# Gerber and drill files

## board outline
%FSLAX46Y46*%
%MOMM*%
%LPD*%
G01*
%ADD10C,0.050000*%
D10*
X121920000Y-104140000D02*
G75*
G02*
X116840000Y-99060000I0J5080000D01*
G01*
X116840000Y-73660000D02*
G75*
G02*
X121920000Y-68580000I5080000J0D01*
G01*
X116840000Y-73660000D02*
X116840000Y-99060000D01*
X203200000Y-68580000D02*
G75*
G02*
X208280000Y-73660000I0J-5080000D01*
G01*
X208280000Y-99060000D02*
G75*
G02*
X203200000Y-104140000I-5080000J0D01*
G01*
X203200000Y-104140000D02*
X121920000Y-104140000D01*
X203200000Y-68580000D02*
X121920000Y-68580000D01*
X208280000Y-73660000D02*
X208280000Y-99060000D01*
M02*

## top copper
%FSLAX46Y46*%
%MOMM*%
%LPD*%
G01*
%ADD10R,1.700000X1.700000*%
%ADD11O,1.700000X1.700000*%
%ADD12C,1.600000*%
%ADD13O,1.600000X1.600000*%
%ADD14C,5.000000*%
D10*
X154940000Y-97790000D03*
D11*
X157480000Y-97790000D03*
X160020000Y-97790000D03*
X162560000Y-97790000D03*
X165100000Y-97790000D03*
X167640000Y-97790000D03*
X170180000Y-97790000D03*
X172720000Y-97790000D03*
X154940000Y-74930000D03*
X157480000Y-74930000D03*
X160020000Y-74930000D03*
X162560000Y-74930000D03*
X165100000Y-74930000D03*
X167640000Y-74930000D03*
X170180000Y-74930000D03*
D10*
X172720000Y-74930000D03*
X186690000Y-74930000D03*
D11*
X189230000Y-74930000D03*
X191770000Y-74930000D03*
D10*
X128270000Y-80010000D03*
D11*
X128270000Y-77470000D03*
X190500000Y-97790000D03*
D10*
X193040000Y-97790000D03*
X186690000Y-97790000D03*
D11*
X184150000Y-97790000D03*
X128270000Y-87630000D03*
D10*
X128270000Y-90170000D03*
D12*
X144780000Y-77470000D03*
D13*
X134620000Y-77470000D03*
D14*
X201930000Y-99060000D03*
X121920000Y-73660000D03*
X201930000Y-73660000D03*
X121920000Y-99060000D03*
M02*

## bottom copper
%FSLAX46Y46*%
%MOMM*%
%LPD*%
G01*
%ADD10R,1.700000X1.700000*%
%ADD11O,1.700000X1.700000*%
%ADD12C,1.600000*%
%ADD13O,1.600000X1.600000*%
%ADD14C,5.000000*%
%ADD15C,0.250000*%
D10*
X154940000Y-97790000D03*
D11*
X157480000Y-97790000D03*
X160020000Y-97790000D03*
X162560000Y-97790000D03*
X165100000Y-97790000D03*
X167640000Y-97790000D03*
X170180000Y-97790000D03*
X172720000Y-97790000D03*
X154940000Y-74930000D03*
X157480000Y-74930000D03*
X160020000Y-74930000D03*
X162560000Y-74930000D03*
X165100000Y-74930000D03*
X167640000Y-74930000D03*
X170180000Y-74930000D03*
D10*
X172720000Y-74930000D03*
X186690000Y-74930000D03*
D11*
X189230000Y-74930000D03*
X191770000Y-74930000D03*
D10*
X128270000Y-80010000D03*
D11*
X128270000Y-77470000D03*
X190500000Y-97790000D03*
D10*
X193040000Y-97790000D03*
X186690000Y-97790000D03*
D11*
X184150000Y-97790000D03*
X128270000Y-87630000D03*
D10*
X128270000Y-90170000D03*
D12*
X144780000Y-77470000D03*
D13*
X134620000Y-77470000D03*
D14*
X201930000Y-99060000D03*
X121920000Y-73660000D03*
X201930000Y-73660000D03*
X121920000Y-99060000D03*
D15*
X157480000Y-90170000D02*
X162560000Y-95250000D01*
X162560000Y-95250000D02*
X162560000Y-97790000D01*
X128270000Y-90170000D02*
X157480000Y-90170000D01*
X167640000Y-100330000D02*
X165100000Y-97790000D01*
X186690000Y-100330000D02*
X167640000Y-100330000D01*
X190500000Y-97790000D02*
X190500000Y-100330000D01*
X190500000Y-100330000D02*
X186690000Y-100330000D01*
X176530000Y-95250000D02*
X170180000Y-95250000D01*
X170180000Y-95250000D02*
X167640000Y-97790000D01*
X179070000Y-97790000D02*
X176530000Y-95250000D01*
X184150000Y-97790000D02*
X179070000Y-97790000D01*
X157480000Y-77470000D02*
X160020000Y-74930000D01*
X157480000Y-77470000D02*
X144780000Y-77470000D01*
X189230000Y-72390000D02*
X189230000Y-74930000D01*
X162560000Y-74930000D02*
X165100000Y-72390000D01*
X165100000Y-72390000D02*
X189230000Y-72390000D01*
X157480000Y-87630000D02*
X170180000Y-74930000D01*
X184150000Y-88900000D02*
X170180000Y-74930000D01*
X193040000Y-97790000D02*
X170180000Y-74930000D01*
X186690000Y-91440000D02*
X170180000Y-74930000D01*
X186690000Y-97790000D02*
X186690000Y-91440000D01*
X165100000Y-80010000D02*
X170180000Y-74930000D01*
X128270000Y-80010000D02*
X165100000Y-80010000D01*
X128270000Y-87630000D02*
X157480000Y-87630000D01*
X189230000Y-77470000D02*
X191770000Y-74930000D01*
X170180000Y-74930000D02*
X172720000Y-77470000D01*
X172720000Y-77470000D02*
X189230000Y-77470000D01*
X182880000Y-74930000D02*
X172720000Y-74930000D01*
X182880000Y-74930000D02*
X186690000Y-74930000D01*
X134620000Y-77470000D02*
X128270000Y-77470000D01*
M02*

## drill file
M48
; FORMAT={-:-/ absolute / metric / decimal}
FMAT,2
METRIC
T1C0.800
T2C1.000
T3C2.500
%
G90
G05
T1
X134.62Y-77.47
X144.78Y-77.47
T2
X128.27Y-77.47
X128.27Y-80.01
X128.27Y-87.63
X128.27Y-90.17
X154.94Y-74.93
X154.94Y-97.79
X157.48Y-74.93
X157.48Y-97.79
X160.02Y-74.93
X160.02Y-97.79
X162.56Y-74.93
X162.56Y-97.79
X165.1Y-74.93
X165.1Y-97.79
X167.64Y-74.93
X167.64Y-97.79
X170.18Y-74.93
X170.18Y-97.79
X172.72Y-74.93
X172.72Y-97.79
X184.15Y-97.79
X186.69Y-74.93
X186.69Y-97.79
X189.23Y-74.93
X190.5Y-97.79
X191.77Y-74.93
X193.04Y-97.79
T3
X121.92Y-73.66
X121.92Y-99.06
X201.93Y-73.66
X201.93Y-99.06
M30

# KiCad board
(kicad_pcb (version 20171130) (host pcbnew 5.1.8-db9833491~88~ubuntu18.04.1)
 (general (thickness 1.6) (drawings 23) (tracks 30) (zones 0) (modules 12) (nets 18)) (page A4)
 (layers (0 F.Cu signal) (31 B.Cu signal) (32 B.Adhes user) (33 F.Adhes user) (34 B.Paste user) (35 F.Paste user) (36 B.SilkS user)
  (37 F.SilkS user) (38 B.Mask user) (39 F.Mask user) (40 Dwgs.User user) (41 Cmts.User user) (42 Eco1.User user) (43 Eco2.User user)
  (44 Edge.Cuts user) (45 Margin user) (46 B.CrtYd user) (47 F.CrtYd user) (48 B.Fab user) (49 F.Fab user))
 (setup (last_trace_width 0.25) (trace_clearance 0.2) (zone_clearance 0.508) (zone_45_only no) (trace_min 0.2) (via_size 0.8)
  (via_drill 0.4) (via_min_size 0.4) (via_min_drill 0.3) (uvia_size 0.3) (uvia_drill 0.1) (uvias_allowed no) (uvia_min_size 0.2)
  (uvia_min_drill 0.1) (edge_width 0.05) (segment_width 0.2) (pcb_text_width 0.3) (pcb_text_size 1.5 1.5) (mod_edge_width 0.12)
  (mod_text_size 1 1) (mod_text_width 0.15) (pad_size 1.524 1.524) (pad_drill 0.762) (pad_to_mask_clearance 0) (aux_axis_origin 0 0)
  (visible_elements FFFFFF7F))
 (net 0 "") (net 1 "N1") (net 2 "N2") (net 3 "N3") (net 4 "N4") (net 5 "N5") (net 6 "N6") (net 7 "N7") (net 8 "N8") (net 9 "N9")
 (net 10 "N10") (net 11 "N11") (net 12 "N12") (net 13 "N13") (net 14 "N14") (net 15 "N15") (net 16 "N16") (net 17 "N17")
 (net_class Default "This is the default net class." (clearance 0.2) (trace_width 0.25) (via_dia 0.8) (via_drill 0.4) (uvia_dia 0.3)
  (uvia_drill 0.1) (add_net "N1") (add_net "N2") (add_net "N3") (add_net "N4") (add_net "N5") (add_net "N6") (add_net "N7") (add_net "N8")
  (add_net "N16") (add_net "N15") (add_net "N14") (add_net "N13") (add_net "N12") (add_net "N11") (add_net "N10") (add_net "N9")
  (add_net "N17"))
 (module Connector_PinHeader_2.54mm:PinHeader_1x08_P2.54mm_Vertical (layer F.Cu) (at 154.94 97.79 90)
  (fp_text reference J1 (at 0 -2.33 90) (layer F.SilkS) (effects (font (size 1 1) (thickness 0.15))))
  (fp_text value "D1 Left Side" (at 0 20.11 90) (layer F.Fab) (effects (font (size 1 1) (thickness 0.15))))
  (pad 1 thru_hole rect (at 0 0 90) (size 1.7 1.7) (drill 1) (layers *.Cu *.Mask) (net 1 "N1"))
  (pad 2 thru_hole oval (at 0 2.54 90) (size 1.7 1.7) (drill 1) (layers *.Cu *.Mask) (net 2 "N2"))
  (pad 3 thru_hole oval (at 0 5.08 90) (size 1.7 1.7) (drill 1) (layers *.Cu *.Mask) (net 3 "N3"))
  (pad 4 thru_hole oval (at 0 7.62 90) (size 1.7 1.7) (drill 1) (layers *.Cu *.Mask) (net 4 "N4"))
  (pad 5 thru_hole oval (at 0 10.16 90) (size 1.7 1.7) (drill 1) (layers *.Cu *.Mask) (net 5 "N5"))
  (pad 6 thru_hole oval (at 0 12.7 90) (size 1.7 1.7) (drill 1) (layers *.Cu *.Mask) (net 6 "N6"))
  (pad 7 thru_hole oval (at 0 15.24 90) (size 1.7 1.7) (drill 1) (layers *.Cu *.Mask) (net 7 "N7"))
  (pad 8 thru_hole oval (at 0 17.78 90) (size 1.7 1.7) (drill 1) (layers *.Cu *.Mask) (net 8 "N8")))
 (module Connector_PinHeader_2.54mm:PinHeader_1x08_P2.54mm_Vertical (layer F.Cu) (at 172.72 74.93 270)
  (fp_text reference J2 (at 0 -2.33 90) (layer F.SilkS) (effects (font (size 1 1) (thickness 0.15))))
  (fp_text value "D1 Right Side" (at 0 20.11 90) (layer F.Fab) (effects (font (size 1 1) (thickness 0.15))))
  (pad 8 thru_hole oval (at 0 17.78 270) (size 1.7 1.7) (drill 1) (layers *.Cu *.Mask) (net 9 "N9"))
  (pad 7 thru_hole oval (at 0 15.24 270) (size 1.7 1.7) (drill 1) (layers *.Cu *.Mask) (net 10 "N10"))
  (pad 6 thru_hole oval (at 0 12.7 270) (size 1.7 1.7) (drill 1) (layers *.Cu *.Mask) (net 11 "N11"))
  (pad 5 thru_hole oval (at 0 10.16 270) (size 1.7 1.7) (drill 1) (layers *.Cu *.Mask) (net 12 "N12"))
  (pad 4 thru_hole oval (at 0 7.62 270) (size 1.7 1.7) (drill 1) (layers *.Cu *.Mask) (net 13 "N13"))
  (pad 3 thru_hole oval (at 0 5.08 270) (size 1.7 1.7) (drill 1) (layers *.Cu *.Mask) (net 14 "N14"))
  (pad 2 thru_hole oval (at 0 2.54 270) (size 1.7 1.7) (drill 1) (layers *.Cu *.Mask) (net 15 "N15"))
  (pad 1 thru_hole rect (at 0 0 270) (size 1.7 1.7) (drill 1) (layers *.Cu *.Mask) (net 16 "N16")))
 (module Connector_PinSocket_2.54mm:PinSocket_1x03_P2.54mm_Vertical (layer F.Cu) (at 186.69 74.93 90)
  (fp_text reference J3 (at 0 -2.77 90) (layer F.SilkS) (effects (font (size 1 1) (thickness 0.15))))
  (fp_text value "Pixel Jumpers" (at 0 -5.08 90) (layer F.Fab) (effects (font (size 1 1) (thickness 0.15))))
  (pad 1 thru_hole rect (at 0 0 90) (size 1.7 1.7) (drill 1) (layers *.Cu *.Mask) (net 16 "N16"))
  (pad 2 thru_hole oval (at 0 2.54 90) (size 1.7 1.7) (drill 1) (layers *.Cu *.Mask) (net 12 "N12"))
  (pad 3 thru_hole oval (at 0 5.08 90) (size 1.7 1.7) (drill 1) (layers *.Cu *.Mask) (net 15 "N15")))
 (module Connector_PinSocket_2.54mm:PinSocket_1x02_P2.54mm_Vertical (layer F.Cu) (at 128.27 80.01 180)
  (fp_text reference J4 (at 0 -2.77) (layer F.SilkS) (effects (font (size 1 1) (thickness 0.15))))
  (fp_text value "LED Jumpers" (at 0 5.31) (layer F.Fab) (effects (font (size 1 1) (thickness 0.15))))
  (pad 1 thru_hole rect (at 0 0 180) (size 1.7 1.7) (drill 1) (layers *.Cu *.Mask) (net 15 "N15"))
  (pad 2 thru_hole oval (at 0 2.54 180) (size 1.7 1.7) (drill 1) (layers *.Cu *.Mask) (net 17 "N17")))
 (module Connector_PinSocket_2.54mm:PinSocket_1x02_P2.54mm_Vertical (layer F.Cu) (at 193.04 97.79 270)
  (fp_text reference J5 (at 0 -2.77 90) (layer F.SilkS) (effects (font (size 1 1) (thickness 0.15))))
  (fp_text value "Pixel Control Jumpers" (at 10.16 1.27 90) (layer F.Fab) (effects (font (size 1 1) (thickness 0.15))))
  (pad 2 thru_hole oval (at 0 2.54 270) (size 1.7 1.7) (drill 1) (layers *.Cu *.Mask) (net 5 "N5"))
  (pad 1 thru_hole rect (at 0 0 270) (size 1.7 1.7) (drill 1) (layers *.Cu *.Mask) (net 15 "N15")))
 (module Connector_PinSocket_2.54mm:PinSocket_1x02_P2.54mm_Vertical (layer F.Cu) (at 186.69 97.79 270)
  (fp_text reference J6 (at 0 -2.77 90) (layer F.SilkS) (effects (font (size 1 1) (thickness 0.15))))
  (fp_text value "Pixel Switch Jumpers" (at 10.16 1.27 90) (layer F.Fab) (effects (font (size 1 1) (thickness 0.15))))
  (pad 1 thru_hole rect (at 0 0 270) (size 1.7 1.7) (drill 1) (layers *.Cu *.Mask) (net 15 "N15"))
  (pad 2 thru_hole oval (at 0 2.54 270) (size 1.7 1.7) (drill 1) (layers *.Cu *.Mask) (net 6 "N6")))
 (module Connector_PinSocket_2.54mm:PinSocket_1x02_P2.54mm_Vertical (layer F.Cu) (at 128.27 90.17 180)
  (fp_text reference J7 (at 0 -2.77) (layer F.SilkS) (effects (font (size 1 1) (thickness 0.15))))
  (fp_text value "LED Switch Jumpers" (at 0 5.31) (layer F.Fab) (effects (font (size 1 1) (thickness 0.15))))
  (pad 2 thru_hole oval (at 0 2.54 180) (size 1.7 1.7) (drill 1) (layers *.Cu *.Mask) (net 15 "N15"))
  (pad 1 thru_hole rect (at 0 0 180) (size 1.7 1.7) (drill 1) (layers *.Cu *.Mask) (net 4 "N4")))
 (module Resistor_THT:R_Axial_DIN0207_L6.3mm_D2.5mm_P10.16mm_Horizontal (layer F.Cu) (at 144.78 77.47 180)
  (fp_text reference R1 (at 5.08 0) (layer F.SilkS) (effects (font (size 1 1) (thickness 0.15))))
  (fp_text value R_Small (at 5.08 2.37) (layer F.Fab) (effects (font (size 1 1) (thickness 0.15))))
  (pad 1 thru_hole circle (at 0 0 180) (size 1.6 1.6) (drill 0.8) (layers *.Cu *.Mask) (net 11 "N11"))
  (pad 2 thru_hole oval (at 10.16 0 180) (size 1.6 1.6) (drill 0.8) (layers *.Cu *.Mask) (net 17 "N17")))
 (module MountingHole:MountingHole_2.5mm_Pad (layer F.Cu) (at 201.93 99.06)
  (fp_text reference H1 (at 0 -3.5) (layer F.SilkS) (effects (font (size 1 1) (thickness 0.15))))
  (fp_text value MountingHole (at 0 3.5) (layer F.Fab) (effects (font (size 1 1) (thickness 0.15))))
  (pad 1 thru_hole circle (at 0 0) (size 5 5) (drill 2.5) (layers *.Cu *.Mask)))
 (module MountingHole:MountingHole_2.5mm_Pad (layer F.Cu) (at 121.92 73.66)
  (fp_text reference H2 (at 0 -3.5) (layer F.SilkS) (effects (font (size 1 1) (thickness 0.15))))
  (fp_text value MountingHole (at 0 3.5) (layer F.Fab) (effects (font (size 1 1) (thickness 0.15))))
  (pad 1 thru_hole circle (at 0 0) (size 5 5) (drill 2.5) (layers *.Cu *.Mask)))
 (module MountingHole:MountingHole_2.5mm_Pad (layer F.Cu) (at 201.93 73.66)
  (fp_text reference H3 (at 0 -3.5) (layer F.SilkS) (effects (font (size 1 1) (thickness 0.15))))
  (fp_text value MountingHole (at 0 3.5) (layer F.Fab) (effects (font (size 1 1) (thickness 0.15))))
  (pad 1 thru_hole circle (at 0 0) (size 5 5) (drill 2.5) (layers *.Cu *.Mask)))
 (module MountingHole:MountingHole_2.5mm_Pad (layer F.Cu) (at 121.92 99.06)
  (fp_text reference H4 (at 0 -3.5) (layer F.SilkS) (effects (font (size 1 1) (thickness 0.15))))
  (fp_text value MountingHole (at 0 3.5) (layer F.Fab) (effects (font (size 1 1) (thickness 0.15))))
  (pad 1 thru_hole circle (at 0 0) (size 5 5) (drill 2.5) (layers *.Cu *.Mask)))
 (gr_arc (start 121.92 99.06) (end 116.84 99.06) (angle -90) (layer Edge.Cuts) (width 0.05))
 (gr_arc (start 121.92 73.66) (end 121.92 68.58) (angle -90) (layer Edge.Cuts) (width 0.05))
 (gr_line (start 116.84 73.66) (end 116.84 99.06) (layer Edge.Cuts) (width 0.05))
 (gr_arc (start 203.2 73.66) (end 208.28 73.66) (angle -90) (layer Edge.Cuts) (width 0.05))
 (gr_arc (start 203.2 99.06) (end 203.2 104.14) (angle -90) (layer Edge.Cuts) (width 0.05))
 (gr_line (start 203.2 104.14) (end 121.92 104.14) (layer Edge.Cuts) (width 0.05))
 (gr_line (start 203.2 68.58) (end 121.92 68.58) (layer Edge.Cuts) (width 0.05))
 (gr_line (start 208.28 73.66) (end 208.28 99.06) (layer Edge.Cuts) (width 0.05))
 (segment (start 157.48 90.17) (end 162.56 95.25) (width 0.25) (layer B.Cu) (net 4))
 (segment (start 162.56 95.25) (end 162.56 97.79) (width 0.25) (layer B.Cu) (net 4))
 (segment (start 128.27 90.17) (end 157.48 90.17) (width 0.25) (layer B.Cu) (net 4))
 (segment (start 167.64 100.33) (end 165.1 97.79) (width 0.25) (layer B.Cu) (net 5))
 (segment (start 186.69 100.33) (end 167.64 100.33) (width 0.25) (layer B.Cu) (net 5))
 (segment (start 190.5 97.79) (end 190.5 100.33) (width 0.25) (layer B.Cu) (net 5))
 (segment (start 190.5 100.33) (end 186.69 100.33) (width 0.25) (layer B.Cu) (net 5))
 (segment (start 176.53 95.25) (end 170.18 95.25) (width 0.25) (layer B.Cu) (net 6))
 (segment (start 170.18 95.25) (end 167.64 97.79) (width 0.25) (layer B.Cu) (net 6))
 (segment (start 179.07 97.79) (end 176.53 95.25) (width 0.25) (layer B.Cu) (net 6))
 (segment (start 184.15 97.79) (end 179.07 97.79) (width 0.25) (layer B.Cu) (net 6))
 (segment (start 157.48 77.47) (end 160.02 74.93) (width 0.25) (layer B.Cu) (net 11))
 (segment (start 157.48 77.47) (end 144.78 77.47) (width 0.25) (layer B.Cu) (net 11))
 (segment (start 189.23 72.39) (end 189.23 74.93) (width 0.25) (layer B.Cu) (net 12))
 (segment (start 162.56 74.93) (end 165.1 72.39) (width 0.25) (layer B.Cu) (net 12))
 (segment (start 165.1 72.39) (end 189.23 72.39) (width 0.25) (layer B.Cu) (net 12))
 (segment (start 157.48 87.63) (end 170.18 74.93) (width 0.25) (layer B.Cu) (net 15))
 (segment (start 184.15 88.9) (end 170.18 74.93) (width 0.25) (layer B.Cu) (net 15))
 (segment (start 193.04 97.79) (end 170.18 74.93) (width 0.25) (layer B.Cu) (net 15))
 (segment (start 186.69 91.44) (end 170.18 74.93) (width 0.25) (layer B.Cu) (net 15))
 (segment (start 186.69 97.79) (end 186.69 91.44) (width 0.25) (layer B.Cu) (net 15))
 (segment (start 165.1 80.01) (end 170.18 74.93) (width 0.25) (layer B.Cu) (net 15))
 (segment (start 128.27 80.01) (end 165.1 80.01) (width 0.25) (layer B.Cu) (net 15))
 (segment (start 128.27 87.63) (end 157.48 87.63) (width 0.25) (layer B.Cu) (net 15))
 (segment (start 189.23 77.47) (end 191.77 74.93) (width 0.25) (layer B.Cu) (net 15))
 (segment (start 170.18 74.93) (end 172.72 77.47) (width 0.25) (layer B.Cu) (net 15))
 (segment (start 172.72 77.47) (end 189.23 77.47) (width 0.25) (layer B.Cu) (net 15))
 (segment (start 182.88 74.93) (end 172.72 74.93) (width 0.25) (layer B.Cu) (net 16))
 (segment (start 182.88 74.93) (end 186.69 74.93) (width 0.25) (layer B.Cu) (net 16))
 (segment (start 134.62 77.47) (end 128.27 77.47) (width 0.25) (layer B.Cu) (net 17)))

